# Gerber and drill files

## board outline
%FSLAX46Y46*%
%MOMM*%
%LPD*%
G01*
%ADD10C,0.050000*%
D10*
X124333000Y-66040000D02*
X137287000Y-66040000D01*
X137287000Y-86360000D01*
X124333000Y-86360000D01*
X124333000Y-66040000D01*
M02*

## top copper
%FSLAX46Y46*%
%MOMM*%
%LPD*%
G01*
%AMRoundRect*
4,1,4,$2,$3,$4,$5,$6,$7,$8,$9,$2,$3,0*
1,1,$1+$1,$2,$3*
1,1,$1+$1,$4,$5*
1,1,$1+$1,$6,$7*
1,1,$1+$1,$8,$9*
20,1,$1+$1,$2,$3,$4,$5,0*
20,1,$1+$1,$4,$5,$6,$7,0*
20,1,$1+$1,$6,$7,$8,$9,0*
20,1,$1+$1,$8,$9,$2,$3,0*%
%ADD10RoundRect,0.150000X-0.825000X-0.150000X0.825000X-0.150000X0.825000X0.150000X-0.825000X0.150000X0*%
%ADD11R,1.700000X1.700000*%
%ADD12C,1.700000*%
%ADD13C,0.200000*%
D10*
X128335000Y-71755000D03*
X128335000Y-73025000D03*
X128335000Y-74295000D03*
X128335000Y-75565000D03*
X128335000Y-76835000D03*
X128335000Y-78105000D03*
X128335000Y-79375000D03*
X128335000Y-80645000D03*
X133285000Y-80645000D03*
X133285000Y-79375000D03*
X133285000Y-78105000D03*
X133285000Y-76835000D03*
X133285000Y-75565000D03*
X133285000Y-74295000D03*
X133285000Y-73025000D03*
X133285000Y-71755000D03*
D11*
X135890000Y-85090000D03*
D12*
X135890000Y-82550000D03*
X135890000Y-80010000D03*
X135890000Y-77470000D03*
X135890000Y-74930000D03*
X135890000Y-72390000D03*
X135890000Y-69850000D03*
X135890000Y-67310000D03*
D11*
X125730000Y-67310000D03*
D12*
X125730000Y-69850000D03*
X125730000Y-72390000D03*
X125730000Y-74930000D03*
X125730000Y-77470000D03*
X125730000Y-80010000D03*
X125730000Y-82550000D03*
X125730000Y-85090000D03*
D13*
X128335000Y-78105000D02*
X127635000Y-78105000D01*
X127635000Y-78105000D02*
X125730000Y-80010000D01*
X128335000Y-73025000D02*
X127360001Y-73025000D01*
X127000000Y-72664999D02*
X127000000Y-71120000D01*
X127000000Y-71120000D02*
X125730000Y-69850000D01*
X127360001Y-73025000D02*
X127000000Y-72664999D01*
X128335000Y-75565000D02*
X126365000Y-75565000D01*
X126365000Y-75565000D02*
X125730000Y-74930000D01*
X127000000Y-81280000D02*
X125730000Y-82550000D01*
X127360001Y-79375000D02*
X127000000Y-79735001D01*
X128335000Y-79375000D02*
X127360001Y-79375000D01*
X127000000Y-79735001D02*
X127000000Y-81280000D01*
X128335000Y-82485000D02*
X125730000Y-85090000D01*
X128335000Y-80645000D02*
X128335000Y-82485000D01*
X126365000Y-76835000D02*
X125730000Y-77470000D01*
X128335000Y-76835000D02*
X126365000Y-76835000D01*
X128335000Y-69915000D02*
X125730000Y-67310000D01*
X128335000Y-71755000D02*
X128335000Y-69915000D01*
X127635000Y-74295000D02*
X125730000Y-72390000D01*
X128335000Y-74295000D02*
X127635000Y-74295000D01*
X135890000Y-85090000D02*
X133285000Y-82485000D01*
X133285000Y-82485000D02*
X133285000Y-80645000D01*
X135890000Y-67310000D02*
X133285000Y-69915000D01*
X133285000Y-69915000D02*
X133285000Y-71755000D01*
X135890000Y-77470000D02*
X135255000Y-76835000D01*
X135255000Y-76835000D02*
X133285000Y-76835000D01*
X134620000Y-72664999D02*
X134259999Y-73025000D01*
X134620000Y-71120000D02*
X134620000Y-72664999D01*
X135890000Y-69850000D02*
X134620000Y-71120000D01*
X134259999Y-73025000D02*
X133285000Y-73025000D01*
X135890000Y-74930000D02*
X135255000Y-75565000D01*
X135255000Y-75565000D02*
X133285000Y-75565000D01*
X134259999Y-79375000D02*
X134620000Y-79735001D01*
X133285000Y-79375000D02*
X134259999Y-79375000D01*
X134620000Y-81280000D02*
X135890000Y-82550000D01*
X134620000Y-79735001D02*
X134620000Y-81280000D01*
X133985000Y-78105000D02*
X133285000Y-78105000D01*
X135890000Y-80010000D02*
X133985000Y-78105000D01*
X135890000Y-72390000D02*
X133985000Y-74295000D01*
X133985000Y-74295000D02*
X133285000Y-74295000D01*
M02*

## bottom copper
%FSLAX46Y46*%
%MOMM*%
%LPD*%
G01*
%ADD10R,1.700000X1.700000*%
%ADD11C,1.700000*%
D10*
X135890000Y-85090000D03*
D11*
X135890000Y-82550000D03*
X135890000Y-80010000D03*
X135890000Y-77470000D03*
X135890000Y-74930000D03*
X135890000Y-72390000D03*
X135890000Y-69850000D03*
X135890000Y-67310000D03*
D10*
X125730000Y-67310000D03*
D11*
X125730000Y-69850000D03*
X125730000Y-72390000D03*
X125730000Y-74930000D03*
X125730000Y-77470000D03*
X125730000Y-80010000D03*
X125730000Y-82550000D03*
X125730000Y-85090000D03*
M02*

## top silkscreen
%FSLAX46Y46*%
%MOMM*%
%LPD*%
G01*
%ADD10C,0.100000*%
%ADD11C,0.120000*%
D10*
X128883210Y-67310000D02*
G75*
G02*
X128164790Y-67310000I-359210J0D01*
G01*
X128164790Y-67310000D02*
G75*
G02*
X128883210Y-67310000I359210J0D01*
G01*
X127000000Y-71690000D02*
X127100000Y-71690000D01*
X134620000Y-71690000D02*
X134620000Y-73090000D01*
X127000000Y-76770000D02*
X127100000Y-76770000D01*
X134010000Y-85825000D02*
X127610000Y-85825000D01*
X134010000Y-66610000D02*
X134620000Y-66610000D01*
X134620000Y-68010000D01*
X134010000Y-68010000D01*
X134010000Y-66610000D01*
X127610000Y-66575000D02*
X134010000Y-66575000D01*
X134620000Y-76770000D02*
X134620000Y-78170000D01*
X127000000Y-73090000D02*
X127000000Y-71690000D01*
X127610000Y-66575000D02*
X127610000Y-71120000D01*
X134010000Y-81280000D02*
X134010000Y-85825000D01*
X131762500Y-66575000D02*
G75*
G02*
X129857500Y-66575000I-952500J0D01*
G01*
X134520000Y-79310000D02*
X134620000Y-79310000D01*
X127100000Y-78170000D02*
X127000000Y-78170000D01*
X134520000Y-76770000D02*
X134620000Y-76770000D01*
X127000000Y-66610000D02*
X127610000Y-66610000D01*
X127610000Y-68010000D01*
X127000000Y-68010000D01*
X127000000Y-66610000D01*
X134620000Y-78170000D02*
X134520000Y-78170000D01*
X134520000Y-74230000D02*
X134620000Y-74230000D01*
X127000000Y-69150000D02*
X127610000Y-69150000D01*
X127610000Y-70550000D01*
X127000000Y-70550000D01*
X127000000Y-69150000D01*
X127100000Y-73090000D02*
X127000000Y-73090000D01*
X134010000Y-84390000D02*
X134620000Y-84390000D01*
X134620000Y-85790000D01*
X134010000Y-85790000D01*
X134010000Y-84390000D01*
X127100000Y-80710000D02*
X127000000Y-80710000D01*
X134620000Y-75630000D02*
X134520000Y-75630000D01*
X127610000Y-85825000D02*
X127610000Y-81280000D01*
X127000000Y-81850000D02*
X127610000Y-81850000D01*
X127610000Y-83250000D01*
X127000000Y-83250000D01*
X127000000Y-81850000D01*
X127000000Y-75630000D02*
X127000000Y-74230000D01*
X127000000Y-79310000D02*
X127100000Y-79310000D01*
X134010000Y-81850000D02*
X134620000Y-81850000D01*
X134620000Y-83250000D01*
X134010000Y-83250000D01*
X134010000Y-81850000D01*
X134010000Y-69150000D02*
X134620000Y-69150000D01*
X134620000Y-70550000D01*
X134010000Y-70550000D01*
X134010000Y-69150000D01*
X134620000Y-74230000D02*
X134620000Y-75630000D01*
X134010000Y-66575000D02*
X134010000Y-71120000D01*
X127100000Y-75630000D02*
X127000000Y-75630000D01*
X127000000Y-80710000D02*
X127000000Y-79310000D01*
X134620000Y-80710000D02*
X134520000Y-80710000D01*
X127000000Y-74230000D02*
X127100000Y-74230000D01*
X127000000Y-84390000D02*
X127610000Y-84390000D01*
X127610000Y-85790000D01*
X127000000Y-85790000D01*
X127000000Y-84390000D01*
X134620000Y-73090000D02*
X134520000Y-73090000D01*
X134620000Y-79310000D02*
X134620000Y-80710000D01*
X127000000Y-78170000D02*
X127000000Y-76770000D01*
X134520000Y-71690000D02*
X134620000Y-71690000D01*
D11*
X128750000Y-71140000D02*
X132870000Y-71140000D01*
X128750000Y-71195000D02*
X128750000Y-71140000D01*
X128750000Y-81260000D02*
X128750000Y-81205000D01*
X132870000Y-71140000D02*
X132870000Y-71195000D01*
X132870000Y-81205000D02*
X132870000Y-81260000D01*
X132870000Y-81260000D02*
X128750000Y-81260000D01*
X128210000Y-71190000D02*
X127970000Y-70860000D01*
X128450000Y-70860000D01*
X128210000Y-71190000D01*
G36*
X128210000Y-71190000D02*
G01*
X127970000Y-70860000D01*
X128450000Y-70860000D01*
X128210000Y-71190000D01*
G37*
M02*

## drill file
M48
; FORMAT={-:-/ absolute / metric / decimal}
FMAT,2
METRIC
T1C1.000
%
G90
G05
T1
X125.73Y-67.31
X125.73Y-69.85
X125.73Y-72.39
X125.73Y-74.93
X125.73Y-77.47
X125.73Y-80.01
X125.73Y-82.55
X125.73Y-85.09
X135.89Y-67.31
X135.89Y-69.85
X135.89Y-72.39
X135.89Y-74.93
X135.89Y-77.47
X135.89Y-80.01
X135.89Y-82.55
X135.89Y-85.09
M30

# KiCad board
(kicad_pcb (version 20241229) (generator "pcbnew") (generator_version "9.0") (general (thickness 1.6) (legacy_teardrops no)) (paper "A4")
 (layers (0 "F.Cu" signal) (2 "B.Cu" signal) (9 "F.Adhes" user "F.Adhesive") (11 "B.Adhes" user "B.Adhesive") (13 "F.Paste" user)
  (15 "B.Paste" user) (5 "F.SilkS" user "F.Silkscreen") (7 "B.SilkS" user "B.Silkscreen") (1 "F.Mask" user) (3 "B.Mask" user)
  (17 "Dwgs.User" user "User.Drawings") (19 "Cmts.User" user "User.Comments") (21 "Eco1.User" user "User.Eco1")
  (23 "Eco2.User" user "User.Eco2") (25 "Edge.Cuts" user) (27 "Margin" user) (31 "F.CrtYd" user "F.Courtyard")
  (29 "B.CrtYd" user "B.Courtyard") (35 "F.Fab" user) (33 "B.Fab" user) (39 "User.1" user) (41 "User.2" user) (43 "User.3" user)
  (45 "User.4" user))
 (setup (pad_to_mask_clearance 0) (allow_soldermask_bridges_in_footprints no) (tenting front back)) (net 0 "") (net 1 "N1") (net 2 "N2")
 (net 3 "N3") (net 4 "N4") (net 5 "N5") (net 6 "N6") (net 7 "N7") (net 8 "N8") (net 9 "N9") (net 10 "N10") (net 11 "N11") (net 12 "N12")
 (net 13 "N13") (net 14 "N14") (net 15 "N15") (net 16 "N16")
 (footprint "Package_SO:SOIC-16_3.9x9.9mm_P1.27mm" (layer "F.Cu") (at 130.81 76.2)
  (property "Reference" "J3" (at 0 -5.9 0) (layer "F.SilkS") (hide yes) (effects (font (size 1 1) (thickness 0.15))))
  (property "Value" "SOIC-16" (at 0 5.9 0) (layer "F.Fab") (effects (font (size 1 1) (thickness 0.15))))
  (fp_line (start -2.06 -5.06) (end 2.06 -5.06) (stroke (width 0.12) (type solid)) (layer "F.SilkS"))
  (fp_line (start -2.06 -5.005) (end -2.06 -5.06) (stroke (width 0.12) (type solid)) (layer "F.SilkS"))
  (fp_line (start -2.06 5.06) (end -2.06 5.005) (stroke (width 0.12) (type solid)) (layer "F.SilkS"))
  (fp_line (start 2.06 -5.06) (end 2.06 -5.005) (stroke (width 0.12) (type solid)) (layer "F.SilkS"))
  (fp_line (start 2.06 5.005) (end 2.06 5.06) (stroke (width 0.12) (type solid)) (layer "F.SilkS"))
  (fp_line (start 2.06 5.06) (end -2.06 5.06) (stroke (width 0.12) (type solid)) (layer "F.SilkS"))
  (fp_poly (pts (xy -2.6 -5.01) (xy -2.84 -5.34) (xy -2.36 -5.34)) (stroke (width 0.12) (type solid)) (fill yes) (layer "F.SilkS"))
  (pad "1" smd roundrect (at -2.475 -4.445) (size 1.95 0.6) (layers "F.Cu" "F.Mask" "F.Paste") (roundrect_rratio 0.25) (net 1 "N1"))
  (pad "2" smd roundrect (at -2.475 -3.175) (size 1.95 0.6) (layers "F.Cu" "F.Mask" "F.Paste") (roundrect_rratio 0.25) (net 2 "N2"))
  (pad "3" smd roundrect (at -2.475 -1.905) (size 1.95 0.6) (layers "F.Cu" "F.Mask" "F.Paste") (roundrect_rratio 0.25) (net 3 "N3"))
  (pad "4" smd roundrect (at -2.475 -0.635) (size 1.95 0.6) (layers "F.Cu" "F.Mask" "F.Paste") (roundrect_rratio 0.25) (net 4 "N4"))
  (pad "5" smd roundrect (at -2.475 0.635) (size 1.95 0.6) (layers "F.Cu" "F.Mask" "F.Paste") (roundrect_rratio 0.25) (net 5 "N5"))
  (pad "6" smd roundrect (at -2.475 1.905) (size 1.95 0.6) (layers "F.Cu" "F.Mask" "F.Paste") (roundrect_rratio 0.25) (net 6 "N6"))
  (pad "7" smd roundrect (at -2.475 3.175) (size 1.95 0.6) (layers "F.Cu" "F.Mask" "F.Paste") (roundrect_rratio 0.25) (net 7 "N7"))
  (pad "8" smd roundrect (at -2.475 4.445) (size 1.95 0.6) (layers "F.Cu" "F.Mask" "F.Paste") (roundrect_rratio 0.25) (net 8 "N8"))
  (pad "9" smd roundrect (at 2.475 4.445) (size 1.95 0.6) (layers "F.Cu" "F.Mask" "F.Paste") (roundrect_rratio 0.25) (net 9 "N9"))
  (pad "10" smd roundrect (at 2.475 3.175) (size 1.95 0.6) (layers "F.Cu" "F.Mask" "F.Paste") (roundrect_rratio 0.25) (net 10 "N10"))
  (pad "11" smd roundrect (at 2.475 1.905) (size 1.95 0.6) (layers "F.Cu" "F.Mask" "F.Paste") (roundrect_rratio 0.25) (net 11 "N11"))
  (pad "12" smd roundrect (at 2.475 0.635) (size 1.95 0.6) (layers "F.Cu" "F.Mask" "F.Paste") (roundrect_rratio 0.25) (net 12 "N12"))
  (pad "13" smd roundrect (at 2.475 -0.635) (size 1.95 0.6) (layers "F.Cu" "F.Mask" "F.Paste") (roundrect_rratio 0.25) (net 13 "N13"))
  (pad "14" smd roundrect (at 2.475 -1.905) (size 1.95 0.6) (layers "F.Cu" "F.Mask" "F.Paste") (roundrect_rratio 0.25) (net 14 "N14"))
  (pad "15" smd roundrect (at 2.475 -3.175) (size 1.95 0.6) (layers "F.Cu" "F.Mask" "F.Paste") (roundrect_rratio 0.25) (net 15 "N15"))
  (pad "16" smd roundrect (at 2.475 -4.445) (size 1.95 0.6) (layers "F.Cu" "F.Mask" "F.Paste") (roundrect_rratio 0.25) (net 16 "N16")))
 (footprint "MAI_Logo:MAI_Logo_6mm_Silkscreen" (layer "B.Cu") (at 131.064 81.788 90)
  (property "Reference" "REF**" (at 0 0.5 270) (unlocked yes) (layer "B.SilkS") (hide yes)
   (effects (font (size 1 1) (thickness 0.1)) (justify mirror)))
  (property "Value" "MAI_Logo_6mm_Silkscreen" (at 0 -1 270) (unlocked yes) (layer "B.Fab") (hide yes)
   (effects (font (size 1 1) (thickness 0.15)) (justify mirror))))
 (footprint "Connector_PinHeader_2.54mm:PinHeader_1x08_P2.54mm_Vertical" (layer "B.Cu") (at 135.89 85.09)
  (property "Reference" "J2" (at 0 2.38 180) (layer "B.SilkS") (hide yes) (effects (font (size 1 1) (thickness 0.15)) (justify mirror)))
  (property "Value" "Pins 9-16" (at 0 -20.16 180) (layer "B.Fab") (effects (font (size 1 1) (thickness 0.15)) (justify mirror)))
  (pad "1" thru_hole rect (at 0 0) (size 1.7 1.7) (drill 1) (layers "*.Cu" "*.Mask") (remove_unused_layers no) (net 9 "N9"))
  (pad "2" thru_hole circle (at 0 -2.54) (size 1.7 1.7) (drill 1) (layers "*.Cu" "*.Mask") (remove_unused_layers no) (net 10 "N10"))
  (pad "3" thru_hole circle (at 0 -5.08) (size 1.7 1.7) (drill 1) (layers "*.Cu" "*.Mask") (remove_unused_layers no) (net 11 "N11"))
  (pad "4" thru_hole circle (at 0 -7.62) (size 1.7 1.7) (drill 1) (layers "*.Cu" "*.Mask") (remove_unused_layers no) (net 12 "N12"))
  (pad "5" thru_hole circle (at 0 -10.16) (size 1.7 1.7) (drill 1) (layers "*.Cu" "*.Mask") (remove_unused_layers no) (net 13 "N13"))
  (pad "6" thru_hole circle (at 0 -12.7) (size 1.7 1.7) (drill 1) (layers "*.Cu" "*.Mask") (remove_unused_layers no) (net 14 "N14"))
  (pad "7" thru_hole circle (at 0 -15.24) (size 1.7 1.7) (drill 1) (layers "*.Cu" "*.Mask") (remove_unused_layers no) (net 15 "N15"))
  (pad "8" thru_hole circle (at 0 -17.78) (size 1.7 1.7) (drill 1) (layers "*.Cu" "*.Mask") (remove_unused_layers no) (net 16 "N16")))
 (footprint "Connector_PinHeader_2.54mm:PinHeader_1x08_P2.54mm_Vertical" (layer "B.Cu") (at 125.73 67.31 180)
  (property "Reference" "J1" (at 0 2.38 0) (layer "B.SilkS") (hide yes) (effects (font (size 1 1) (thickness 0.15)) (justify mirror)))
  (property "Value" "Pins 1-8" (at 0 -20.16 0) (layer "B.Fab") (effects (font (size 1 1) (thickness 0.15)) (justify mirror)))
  (pad "1" thru_hole rect (at 0 0 180) (size 1.7 1.7) (drill 1) (layers "*.Cu" "*.Mask") (remove_unused_layers no) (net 1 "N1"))
  (pad "2" thru_hole circle (at 0 -2.54 180) (size 1.7 1.7) (drill 1) (layers "*.Cu" "*.Mask") (remove_unused_layers no) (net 2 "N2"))
  (pad "3" thru_hole circle (at 0 -5.08 180) (size 1.7 1.7) (drill 1) (layers "*.Cu" "*.Mask") (remove_unused_layers no) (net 3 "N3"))
  (pad "4" thru_hole circle (at 0 -7.62 180) (size 1.7 1.7) (drill 1) (layers "*.Cu" "*.Mask") (remove_unused_layers no) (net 4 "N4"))
  (pad "5" thru_hole circle (at 0 -10.16 180) (size 1.7 1.7) (drill 1) (layers "*.Cu" "*.Mask") (remove_unused_layers no) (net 5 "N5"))
  (pad "6" thru_hole circle (at 0 -12.7 180) (size 1.7 1.7) (drill 1) (layers "*.Cu" "*.Mask") (remove_unused_layers no) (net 6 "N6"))
  (pad "7" thru_hole circle (at 0 -15.24 180) (size 1.7 1.7) (drill 1) (layers "*.Cu" "*.Mask") (remove_unused_layers no) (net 7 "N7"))
  (pad "8" thru_hole circle (at 0 -17.78 180) (size 1.7 1.7) (drill 1) (layers "*.Cu" "*.Mask") (remove_unused_layers no) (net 8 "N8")))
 (gr_circle (center 128.524 67.31) (end 128.778 67.564) (stroke (width 0.1) (type solid)) (fill no) (layer "F.SilkS"))
 (gr_line (start 127 71.69) (end 127.1 71.69) (stroke (width 0.1) (type default)) (layer "F.SilkS"))
 (gr_line (start 134.62 71.69) (end 134.62 73.09) (stroke (width 0.1) (type default)) (layer "F.SilkS"))
 (gr_line (start 127 76.77) (end 127.1 76.77) (stroke (width 0.1) (type default)) (layer "F.SilkS"))
 (gr_line (start 134.01 85.825) (end 127.61 85.825) (stroke (width 0.1) (type default)) (layer "F.SilkS"))
 (gr_rect (start 134.01 66.61) (end 134.62 68.01) (stroke (width 0.1) (type solid)) (fill no) (layer "F.SilkS"))
 (gr_line (start 127.61 66.575) (end 134.01 66.575) (stroke (width 0.1) (type default)) (layer "F.SilkS"))
 (gr_line (start 134.62 76.77) (end 134.62 78.17) (stroke (width 0.1) (type default)) (layer "F.SilkS"))
 (gr_line (start 127 73.09) (end 127 71.69) (stroke (width 0.1) (type default)) (layer "F.SilkS"))
 (gr_line (start 127.61 66.575) (end 127.61 71.12) (stroke (width 0.1) (type solid)) (layer "F.SilkS"))
 (gr_line (start 134.01 81.28) (end 134.01 85.825) (stroke (width 0.1) (type default)) (layer "F.SilkS"))
 (gr_arc (start 131.7625 66.575) (mid 130.81 67.5275) (end 129.8575 66.575) (stroke (width 0.1) (type solid)) (layer "F.SilkS"))
 (gr_line (start 134.52 79.31) (end 134.62 79.31) (stroke (width 0.1) (type default)) (layer "F.SilkS"))
 (gr_line (start 127.1 78.17) (end 127 78.17) (stroke (width 0.1) (type default)) (layer "F.SilkS"))
 (gr_line (start 134.52 76.77) (end 134.62 76.77) (stroke (width 0.1) (type default)) (layer "F.SilkS"))
 (gr_rect (start 127 66.61) (end 127.61 68.01) (stroke (width 0.1) (type solid)) (fill no) (layer "F.SilkS"))
 (gr_line (start 134.62 78.17) (end 134.52 78.17) (stroke (width 0.1) (type default)) (layer "F.SilkS"))
 (gr_line (start 134.52 74.23) (end 134.62 74.23) (stroke (width 0.1) (type default)) (layer "F.SilkS"))
 (gr_rect (start 127 69.15) (end 127.61 70.55) (stroke (width 0.1) (type solid)) (fill no) (layer "F.SilkS"))
 (gr_line (start 127.1 73.09) (end 127 73.09) (stroke (width 0.1) (type default)) (layer "F.SilkS"))
 (gr_rect (start 134.01 84.39) (end 134.62 85.79) (stroke (width 0.1) (type solid)) (fill no) (layer "F.SilkS"))
 (gr_line (start 127.1 80.71) (end 127 80.71) (stroke (width 0.1) (type default)) (layer "F.SilkS"))
 (gr_line (start 134.62 75.63) (end 134.52 75.63) (stroke (width 0.1) (type default)) (layer "F.SilkS"))
 (gr_line (start 127.61 85.825) (end 127.61 81.28) (stroke (width 0.1) (type default)) (layer "F.SilkS"))
 (gr_rect (start 127 81.85) (end 127.61 83.25) (stroke (width 0.1) (type solid)) (fill no) (layer "F.SilkS"))
 (gr_line (start 127 75.63) (end 127 74.23) (stroke (width 0.1) (type default)) (layer "F.SilkS"))
 (gr_line (start 127 79.31) (end 127.1 79.31) (stroke (width 0.1) (type default)) (layer "F.SilkS"))
 (gr_rect (start 134.01 81.85) (end 134.62 83.25) (stroke (width 0.1) (type solid)) (fill no) (layer "F.SilkS"))
 (gr_rect (start 134.01 69.15) (end 134.62 70.55) (stroke (width 0.1) (type solid)) (fill no) (layer "F.SilkS"))
 (gr_line (start 134.62 74.23) (end 134.62 75.63) (stroke (width 0.1) (type default)) (layer "F.SilkS"))
 (gr_line (start 134.01 66.575) (end 134.01 71.12) (stroke (width 0.1) (type default)) (layer "F.SilkS"))
 (gr_line (start 127.1 75.63) (end 127 75.63) (stroke (width 0.1) (type default)) (layer "F.SilkS"))
 (gr_line (start 127 80.71) (end 127 79.31) (stroke (width 0.1) (type default)) (layer "F.SilkS"))
 (gr_line (start 134.62 80.71) (end 134.52 80.71) (stroke (width 0.1) (type default)) (layer "F.SilkS"))
 (gr_line (start 127 74.23) (end 127.1 74.23) (stroke (width 0.1) (type default)) (layer "F.SilkS"))
 (gr_rect (start 127 84.39) (end 127.61 85.79) (stroke (width 0.1) (type solid)) (fill no) (layer "F.SilkS"))
 (gr_line (start 134.62 73.09) (end 134.52 73.09) (stroke (width 0.1) (type default)) (layer "F.SilkS"))
 (gr_line (start 134.62 79.31) (end 134.62 80.71) (stroke (width 0.1) (type default)) (layer "F.SilkS"))
 (gr_line (start 127 78.17) (end 127 76.77) (stroke (width 0.1) (type default)) (layer "F.SilkS"))
 (gr_line (start 134.52 71.69) (end 134.62 71.69) (stroke (width 0.1) (type default)) (layer "F.SilkS"))
 (gr_rect (start 124.333 66.04) (end 137.287 86.36) (stroke (width 0.05) (type solid)) (fill no) (layer "Edge.Cuts"))
 (segment (start 128.335 78.105) (end 127.635 78.105) (width 0.2) (layer "F.Cu") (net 6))
 (segment (start 127.635 78.105) (end 125.73 80.01) (width 0.2) (layer "F.Cu") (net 6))
 (segment (start 128.335 73.025) (end 127.360001 73.025) (width 0.2) (layer "F.Cu") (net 2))
 (segment (start 127 72.664999) (end 127 71.12) (width 0.2) (layer "F.Cu") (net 2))
 (segment (start 127 71.12) (end 125.73 69.85) (width 0.2) (layer "F.Cu") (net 2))
 (segment (start 127.360001 73.025) (end 127 72.664999) (width 0.2) (layer "F.Cu") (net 2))
 (segment (start 128.335 75.565) (end 126.365 75.565) (width 0.2) (layer "F.Cu") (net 4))
 (segment (start 126.365 75.565) (end 125.73 74.93) (width 0.2) (layer "F.Cu") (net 4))
 (segment (start 127 81.28) (end 125.73 82.55) (width 0.2) (layer "F.Cu") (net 7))
 (segment (start 127.360001 79.375) (end 127 79.735001) (width 0.2) (layer "F.Cu") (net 7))
 (segment (start 128.335 79.375) (end 127.360001 79.375) (width 0.2) (layer "F.Cu") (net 7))
 (segment (start 127 79.735001) (end 127 81.28) (width 0.2) (layer "F.Cu") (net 7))
 (segment (start 128.335 82.485) (end 125.73 85.09) (width 0.2) (layer "F.Cu") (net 8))
 (segment (start 128.335 80.645) (end 128.335 82.485) (width 0.2) (layer "F.Cu") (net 8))
 (segment (start 126.365 76.835) (end 125.73 77.47) (width 0.2) (layer "F.Cu") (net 5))
 (segment (start 128.335 76.835) (end 126.365 76.835) (width 0.2) (layer "F.Cu") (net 5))
 (segment (start 128.335 69.915) (end 125.73 67.31) (width 0.2) (layer "F.Cu") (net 1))
 (segment (start 128.335 71.755) (end 128.335 69.915) (width 0.2) (layer "F.Cu") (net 1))
 (segment (start 127.635 74.295) (end 125.73 72.39) (width 0.2) (layer "F.Cu") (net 3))
 (segment (start 128.335 74.295) (end 127.635 74.295) (width 0.2) (layer "F.Cu") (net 3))
 (segment (start 135.89 85.09) (end 133.285 82.485) (width 0.2) (layer "F.Cu") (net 9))
 (segment (start 133.285 82.485) (end 133.285 80.645) (width 0.2) (layer "F.Cu") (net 9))
 (segment (start 135.89 67.31) (end 133.285 69.915) (width 0.2) (layer "F.Cu") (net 16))
 (segment (start 133.285 69.915) (end 133.285 71.755) (width 0.2) (layer "F.Cu") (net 16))
 (segment (start 135.89 77.47) (end 135.255 76.835) (width 0.2) (layer "F.Cu") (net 12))
 (segment (start 135.255 76.835) (end 133.285 76.835) (width 0.2) (layer "F.Cu") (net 12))
 (segment (start 134.62 72.664999) (end 134.259999 73.025) (width 0.2) (layer "F.Cu") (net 15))
 (segment (start 134.62 71.12) (end 134.62 72.664999) (width 0.2) (layer "F.Cu") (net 15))
 (segment (start 135.89 69.85) (end 134.62 71.12) (width 0.2) (layer "F.Cu") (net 15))
 (segment (start 134.259999 73.025) (end 133.285 73.025) (width 0.2) (layer "F.Cu") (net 15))
 (segment (start 135.89 74.93) (end 135.255 75.565) (width 0.2) (layer "F.Cu") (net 13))
 (segment (start 135.255 75.565) (end 133.285 75.565) (width 0.2) (layer "F.Cu") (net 13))
 (segment (start 134.259999 79.375) (end 134.62 79.735001) (width 0.2) (layer "F.Cu") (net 10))
 (segment (start 133.285 79.375) (end 134.259999 79.375) (width 0.2) (layer "F.Cu") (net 10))
 (segment (start 134.62 81.28) (end 135.89 82.55) (width 0.2) (layer "F.Cu") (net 10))
 (segment (start 134.62 79.735001) (end 134.62 81.28) (width 0.2) (layer "F.Cu") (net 10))
 (segment (start 133.985 78.105) (end 133.285 78.105) (width 0.2) (layer "F.Cu") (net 11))
 (segment (start 135.89 80.01) (end 133.985 78.105) (width 0.2) (layer "F.Cu") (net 11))
 (segment (start 135.89 72.39) (end 133.985 74.295) (width 0.2) (layer "F.Cu") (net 14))
 (segment (start 133.985 74.295) (end 133.285 74.295) (width 0.2) (layer "F.Cu") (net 14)))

